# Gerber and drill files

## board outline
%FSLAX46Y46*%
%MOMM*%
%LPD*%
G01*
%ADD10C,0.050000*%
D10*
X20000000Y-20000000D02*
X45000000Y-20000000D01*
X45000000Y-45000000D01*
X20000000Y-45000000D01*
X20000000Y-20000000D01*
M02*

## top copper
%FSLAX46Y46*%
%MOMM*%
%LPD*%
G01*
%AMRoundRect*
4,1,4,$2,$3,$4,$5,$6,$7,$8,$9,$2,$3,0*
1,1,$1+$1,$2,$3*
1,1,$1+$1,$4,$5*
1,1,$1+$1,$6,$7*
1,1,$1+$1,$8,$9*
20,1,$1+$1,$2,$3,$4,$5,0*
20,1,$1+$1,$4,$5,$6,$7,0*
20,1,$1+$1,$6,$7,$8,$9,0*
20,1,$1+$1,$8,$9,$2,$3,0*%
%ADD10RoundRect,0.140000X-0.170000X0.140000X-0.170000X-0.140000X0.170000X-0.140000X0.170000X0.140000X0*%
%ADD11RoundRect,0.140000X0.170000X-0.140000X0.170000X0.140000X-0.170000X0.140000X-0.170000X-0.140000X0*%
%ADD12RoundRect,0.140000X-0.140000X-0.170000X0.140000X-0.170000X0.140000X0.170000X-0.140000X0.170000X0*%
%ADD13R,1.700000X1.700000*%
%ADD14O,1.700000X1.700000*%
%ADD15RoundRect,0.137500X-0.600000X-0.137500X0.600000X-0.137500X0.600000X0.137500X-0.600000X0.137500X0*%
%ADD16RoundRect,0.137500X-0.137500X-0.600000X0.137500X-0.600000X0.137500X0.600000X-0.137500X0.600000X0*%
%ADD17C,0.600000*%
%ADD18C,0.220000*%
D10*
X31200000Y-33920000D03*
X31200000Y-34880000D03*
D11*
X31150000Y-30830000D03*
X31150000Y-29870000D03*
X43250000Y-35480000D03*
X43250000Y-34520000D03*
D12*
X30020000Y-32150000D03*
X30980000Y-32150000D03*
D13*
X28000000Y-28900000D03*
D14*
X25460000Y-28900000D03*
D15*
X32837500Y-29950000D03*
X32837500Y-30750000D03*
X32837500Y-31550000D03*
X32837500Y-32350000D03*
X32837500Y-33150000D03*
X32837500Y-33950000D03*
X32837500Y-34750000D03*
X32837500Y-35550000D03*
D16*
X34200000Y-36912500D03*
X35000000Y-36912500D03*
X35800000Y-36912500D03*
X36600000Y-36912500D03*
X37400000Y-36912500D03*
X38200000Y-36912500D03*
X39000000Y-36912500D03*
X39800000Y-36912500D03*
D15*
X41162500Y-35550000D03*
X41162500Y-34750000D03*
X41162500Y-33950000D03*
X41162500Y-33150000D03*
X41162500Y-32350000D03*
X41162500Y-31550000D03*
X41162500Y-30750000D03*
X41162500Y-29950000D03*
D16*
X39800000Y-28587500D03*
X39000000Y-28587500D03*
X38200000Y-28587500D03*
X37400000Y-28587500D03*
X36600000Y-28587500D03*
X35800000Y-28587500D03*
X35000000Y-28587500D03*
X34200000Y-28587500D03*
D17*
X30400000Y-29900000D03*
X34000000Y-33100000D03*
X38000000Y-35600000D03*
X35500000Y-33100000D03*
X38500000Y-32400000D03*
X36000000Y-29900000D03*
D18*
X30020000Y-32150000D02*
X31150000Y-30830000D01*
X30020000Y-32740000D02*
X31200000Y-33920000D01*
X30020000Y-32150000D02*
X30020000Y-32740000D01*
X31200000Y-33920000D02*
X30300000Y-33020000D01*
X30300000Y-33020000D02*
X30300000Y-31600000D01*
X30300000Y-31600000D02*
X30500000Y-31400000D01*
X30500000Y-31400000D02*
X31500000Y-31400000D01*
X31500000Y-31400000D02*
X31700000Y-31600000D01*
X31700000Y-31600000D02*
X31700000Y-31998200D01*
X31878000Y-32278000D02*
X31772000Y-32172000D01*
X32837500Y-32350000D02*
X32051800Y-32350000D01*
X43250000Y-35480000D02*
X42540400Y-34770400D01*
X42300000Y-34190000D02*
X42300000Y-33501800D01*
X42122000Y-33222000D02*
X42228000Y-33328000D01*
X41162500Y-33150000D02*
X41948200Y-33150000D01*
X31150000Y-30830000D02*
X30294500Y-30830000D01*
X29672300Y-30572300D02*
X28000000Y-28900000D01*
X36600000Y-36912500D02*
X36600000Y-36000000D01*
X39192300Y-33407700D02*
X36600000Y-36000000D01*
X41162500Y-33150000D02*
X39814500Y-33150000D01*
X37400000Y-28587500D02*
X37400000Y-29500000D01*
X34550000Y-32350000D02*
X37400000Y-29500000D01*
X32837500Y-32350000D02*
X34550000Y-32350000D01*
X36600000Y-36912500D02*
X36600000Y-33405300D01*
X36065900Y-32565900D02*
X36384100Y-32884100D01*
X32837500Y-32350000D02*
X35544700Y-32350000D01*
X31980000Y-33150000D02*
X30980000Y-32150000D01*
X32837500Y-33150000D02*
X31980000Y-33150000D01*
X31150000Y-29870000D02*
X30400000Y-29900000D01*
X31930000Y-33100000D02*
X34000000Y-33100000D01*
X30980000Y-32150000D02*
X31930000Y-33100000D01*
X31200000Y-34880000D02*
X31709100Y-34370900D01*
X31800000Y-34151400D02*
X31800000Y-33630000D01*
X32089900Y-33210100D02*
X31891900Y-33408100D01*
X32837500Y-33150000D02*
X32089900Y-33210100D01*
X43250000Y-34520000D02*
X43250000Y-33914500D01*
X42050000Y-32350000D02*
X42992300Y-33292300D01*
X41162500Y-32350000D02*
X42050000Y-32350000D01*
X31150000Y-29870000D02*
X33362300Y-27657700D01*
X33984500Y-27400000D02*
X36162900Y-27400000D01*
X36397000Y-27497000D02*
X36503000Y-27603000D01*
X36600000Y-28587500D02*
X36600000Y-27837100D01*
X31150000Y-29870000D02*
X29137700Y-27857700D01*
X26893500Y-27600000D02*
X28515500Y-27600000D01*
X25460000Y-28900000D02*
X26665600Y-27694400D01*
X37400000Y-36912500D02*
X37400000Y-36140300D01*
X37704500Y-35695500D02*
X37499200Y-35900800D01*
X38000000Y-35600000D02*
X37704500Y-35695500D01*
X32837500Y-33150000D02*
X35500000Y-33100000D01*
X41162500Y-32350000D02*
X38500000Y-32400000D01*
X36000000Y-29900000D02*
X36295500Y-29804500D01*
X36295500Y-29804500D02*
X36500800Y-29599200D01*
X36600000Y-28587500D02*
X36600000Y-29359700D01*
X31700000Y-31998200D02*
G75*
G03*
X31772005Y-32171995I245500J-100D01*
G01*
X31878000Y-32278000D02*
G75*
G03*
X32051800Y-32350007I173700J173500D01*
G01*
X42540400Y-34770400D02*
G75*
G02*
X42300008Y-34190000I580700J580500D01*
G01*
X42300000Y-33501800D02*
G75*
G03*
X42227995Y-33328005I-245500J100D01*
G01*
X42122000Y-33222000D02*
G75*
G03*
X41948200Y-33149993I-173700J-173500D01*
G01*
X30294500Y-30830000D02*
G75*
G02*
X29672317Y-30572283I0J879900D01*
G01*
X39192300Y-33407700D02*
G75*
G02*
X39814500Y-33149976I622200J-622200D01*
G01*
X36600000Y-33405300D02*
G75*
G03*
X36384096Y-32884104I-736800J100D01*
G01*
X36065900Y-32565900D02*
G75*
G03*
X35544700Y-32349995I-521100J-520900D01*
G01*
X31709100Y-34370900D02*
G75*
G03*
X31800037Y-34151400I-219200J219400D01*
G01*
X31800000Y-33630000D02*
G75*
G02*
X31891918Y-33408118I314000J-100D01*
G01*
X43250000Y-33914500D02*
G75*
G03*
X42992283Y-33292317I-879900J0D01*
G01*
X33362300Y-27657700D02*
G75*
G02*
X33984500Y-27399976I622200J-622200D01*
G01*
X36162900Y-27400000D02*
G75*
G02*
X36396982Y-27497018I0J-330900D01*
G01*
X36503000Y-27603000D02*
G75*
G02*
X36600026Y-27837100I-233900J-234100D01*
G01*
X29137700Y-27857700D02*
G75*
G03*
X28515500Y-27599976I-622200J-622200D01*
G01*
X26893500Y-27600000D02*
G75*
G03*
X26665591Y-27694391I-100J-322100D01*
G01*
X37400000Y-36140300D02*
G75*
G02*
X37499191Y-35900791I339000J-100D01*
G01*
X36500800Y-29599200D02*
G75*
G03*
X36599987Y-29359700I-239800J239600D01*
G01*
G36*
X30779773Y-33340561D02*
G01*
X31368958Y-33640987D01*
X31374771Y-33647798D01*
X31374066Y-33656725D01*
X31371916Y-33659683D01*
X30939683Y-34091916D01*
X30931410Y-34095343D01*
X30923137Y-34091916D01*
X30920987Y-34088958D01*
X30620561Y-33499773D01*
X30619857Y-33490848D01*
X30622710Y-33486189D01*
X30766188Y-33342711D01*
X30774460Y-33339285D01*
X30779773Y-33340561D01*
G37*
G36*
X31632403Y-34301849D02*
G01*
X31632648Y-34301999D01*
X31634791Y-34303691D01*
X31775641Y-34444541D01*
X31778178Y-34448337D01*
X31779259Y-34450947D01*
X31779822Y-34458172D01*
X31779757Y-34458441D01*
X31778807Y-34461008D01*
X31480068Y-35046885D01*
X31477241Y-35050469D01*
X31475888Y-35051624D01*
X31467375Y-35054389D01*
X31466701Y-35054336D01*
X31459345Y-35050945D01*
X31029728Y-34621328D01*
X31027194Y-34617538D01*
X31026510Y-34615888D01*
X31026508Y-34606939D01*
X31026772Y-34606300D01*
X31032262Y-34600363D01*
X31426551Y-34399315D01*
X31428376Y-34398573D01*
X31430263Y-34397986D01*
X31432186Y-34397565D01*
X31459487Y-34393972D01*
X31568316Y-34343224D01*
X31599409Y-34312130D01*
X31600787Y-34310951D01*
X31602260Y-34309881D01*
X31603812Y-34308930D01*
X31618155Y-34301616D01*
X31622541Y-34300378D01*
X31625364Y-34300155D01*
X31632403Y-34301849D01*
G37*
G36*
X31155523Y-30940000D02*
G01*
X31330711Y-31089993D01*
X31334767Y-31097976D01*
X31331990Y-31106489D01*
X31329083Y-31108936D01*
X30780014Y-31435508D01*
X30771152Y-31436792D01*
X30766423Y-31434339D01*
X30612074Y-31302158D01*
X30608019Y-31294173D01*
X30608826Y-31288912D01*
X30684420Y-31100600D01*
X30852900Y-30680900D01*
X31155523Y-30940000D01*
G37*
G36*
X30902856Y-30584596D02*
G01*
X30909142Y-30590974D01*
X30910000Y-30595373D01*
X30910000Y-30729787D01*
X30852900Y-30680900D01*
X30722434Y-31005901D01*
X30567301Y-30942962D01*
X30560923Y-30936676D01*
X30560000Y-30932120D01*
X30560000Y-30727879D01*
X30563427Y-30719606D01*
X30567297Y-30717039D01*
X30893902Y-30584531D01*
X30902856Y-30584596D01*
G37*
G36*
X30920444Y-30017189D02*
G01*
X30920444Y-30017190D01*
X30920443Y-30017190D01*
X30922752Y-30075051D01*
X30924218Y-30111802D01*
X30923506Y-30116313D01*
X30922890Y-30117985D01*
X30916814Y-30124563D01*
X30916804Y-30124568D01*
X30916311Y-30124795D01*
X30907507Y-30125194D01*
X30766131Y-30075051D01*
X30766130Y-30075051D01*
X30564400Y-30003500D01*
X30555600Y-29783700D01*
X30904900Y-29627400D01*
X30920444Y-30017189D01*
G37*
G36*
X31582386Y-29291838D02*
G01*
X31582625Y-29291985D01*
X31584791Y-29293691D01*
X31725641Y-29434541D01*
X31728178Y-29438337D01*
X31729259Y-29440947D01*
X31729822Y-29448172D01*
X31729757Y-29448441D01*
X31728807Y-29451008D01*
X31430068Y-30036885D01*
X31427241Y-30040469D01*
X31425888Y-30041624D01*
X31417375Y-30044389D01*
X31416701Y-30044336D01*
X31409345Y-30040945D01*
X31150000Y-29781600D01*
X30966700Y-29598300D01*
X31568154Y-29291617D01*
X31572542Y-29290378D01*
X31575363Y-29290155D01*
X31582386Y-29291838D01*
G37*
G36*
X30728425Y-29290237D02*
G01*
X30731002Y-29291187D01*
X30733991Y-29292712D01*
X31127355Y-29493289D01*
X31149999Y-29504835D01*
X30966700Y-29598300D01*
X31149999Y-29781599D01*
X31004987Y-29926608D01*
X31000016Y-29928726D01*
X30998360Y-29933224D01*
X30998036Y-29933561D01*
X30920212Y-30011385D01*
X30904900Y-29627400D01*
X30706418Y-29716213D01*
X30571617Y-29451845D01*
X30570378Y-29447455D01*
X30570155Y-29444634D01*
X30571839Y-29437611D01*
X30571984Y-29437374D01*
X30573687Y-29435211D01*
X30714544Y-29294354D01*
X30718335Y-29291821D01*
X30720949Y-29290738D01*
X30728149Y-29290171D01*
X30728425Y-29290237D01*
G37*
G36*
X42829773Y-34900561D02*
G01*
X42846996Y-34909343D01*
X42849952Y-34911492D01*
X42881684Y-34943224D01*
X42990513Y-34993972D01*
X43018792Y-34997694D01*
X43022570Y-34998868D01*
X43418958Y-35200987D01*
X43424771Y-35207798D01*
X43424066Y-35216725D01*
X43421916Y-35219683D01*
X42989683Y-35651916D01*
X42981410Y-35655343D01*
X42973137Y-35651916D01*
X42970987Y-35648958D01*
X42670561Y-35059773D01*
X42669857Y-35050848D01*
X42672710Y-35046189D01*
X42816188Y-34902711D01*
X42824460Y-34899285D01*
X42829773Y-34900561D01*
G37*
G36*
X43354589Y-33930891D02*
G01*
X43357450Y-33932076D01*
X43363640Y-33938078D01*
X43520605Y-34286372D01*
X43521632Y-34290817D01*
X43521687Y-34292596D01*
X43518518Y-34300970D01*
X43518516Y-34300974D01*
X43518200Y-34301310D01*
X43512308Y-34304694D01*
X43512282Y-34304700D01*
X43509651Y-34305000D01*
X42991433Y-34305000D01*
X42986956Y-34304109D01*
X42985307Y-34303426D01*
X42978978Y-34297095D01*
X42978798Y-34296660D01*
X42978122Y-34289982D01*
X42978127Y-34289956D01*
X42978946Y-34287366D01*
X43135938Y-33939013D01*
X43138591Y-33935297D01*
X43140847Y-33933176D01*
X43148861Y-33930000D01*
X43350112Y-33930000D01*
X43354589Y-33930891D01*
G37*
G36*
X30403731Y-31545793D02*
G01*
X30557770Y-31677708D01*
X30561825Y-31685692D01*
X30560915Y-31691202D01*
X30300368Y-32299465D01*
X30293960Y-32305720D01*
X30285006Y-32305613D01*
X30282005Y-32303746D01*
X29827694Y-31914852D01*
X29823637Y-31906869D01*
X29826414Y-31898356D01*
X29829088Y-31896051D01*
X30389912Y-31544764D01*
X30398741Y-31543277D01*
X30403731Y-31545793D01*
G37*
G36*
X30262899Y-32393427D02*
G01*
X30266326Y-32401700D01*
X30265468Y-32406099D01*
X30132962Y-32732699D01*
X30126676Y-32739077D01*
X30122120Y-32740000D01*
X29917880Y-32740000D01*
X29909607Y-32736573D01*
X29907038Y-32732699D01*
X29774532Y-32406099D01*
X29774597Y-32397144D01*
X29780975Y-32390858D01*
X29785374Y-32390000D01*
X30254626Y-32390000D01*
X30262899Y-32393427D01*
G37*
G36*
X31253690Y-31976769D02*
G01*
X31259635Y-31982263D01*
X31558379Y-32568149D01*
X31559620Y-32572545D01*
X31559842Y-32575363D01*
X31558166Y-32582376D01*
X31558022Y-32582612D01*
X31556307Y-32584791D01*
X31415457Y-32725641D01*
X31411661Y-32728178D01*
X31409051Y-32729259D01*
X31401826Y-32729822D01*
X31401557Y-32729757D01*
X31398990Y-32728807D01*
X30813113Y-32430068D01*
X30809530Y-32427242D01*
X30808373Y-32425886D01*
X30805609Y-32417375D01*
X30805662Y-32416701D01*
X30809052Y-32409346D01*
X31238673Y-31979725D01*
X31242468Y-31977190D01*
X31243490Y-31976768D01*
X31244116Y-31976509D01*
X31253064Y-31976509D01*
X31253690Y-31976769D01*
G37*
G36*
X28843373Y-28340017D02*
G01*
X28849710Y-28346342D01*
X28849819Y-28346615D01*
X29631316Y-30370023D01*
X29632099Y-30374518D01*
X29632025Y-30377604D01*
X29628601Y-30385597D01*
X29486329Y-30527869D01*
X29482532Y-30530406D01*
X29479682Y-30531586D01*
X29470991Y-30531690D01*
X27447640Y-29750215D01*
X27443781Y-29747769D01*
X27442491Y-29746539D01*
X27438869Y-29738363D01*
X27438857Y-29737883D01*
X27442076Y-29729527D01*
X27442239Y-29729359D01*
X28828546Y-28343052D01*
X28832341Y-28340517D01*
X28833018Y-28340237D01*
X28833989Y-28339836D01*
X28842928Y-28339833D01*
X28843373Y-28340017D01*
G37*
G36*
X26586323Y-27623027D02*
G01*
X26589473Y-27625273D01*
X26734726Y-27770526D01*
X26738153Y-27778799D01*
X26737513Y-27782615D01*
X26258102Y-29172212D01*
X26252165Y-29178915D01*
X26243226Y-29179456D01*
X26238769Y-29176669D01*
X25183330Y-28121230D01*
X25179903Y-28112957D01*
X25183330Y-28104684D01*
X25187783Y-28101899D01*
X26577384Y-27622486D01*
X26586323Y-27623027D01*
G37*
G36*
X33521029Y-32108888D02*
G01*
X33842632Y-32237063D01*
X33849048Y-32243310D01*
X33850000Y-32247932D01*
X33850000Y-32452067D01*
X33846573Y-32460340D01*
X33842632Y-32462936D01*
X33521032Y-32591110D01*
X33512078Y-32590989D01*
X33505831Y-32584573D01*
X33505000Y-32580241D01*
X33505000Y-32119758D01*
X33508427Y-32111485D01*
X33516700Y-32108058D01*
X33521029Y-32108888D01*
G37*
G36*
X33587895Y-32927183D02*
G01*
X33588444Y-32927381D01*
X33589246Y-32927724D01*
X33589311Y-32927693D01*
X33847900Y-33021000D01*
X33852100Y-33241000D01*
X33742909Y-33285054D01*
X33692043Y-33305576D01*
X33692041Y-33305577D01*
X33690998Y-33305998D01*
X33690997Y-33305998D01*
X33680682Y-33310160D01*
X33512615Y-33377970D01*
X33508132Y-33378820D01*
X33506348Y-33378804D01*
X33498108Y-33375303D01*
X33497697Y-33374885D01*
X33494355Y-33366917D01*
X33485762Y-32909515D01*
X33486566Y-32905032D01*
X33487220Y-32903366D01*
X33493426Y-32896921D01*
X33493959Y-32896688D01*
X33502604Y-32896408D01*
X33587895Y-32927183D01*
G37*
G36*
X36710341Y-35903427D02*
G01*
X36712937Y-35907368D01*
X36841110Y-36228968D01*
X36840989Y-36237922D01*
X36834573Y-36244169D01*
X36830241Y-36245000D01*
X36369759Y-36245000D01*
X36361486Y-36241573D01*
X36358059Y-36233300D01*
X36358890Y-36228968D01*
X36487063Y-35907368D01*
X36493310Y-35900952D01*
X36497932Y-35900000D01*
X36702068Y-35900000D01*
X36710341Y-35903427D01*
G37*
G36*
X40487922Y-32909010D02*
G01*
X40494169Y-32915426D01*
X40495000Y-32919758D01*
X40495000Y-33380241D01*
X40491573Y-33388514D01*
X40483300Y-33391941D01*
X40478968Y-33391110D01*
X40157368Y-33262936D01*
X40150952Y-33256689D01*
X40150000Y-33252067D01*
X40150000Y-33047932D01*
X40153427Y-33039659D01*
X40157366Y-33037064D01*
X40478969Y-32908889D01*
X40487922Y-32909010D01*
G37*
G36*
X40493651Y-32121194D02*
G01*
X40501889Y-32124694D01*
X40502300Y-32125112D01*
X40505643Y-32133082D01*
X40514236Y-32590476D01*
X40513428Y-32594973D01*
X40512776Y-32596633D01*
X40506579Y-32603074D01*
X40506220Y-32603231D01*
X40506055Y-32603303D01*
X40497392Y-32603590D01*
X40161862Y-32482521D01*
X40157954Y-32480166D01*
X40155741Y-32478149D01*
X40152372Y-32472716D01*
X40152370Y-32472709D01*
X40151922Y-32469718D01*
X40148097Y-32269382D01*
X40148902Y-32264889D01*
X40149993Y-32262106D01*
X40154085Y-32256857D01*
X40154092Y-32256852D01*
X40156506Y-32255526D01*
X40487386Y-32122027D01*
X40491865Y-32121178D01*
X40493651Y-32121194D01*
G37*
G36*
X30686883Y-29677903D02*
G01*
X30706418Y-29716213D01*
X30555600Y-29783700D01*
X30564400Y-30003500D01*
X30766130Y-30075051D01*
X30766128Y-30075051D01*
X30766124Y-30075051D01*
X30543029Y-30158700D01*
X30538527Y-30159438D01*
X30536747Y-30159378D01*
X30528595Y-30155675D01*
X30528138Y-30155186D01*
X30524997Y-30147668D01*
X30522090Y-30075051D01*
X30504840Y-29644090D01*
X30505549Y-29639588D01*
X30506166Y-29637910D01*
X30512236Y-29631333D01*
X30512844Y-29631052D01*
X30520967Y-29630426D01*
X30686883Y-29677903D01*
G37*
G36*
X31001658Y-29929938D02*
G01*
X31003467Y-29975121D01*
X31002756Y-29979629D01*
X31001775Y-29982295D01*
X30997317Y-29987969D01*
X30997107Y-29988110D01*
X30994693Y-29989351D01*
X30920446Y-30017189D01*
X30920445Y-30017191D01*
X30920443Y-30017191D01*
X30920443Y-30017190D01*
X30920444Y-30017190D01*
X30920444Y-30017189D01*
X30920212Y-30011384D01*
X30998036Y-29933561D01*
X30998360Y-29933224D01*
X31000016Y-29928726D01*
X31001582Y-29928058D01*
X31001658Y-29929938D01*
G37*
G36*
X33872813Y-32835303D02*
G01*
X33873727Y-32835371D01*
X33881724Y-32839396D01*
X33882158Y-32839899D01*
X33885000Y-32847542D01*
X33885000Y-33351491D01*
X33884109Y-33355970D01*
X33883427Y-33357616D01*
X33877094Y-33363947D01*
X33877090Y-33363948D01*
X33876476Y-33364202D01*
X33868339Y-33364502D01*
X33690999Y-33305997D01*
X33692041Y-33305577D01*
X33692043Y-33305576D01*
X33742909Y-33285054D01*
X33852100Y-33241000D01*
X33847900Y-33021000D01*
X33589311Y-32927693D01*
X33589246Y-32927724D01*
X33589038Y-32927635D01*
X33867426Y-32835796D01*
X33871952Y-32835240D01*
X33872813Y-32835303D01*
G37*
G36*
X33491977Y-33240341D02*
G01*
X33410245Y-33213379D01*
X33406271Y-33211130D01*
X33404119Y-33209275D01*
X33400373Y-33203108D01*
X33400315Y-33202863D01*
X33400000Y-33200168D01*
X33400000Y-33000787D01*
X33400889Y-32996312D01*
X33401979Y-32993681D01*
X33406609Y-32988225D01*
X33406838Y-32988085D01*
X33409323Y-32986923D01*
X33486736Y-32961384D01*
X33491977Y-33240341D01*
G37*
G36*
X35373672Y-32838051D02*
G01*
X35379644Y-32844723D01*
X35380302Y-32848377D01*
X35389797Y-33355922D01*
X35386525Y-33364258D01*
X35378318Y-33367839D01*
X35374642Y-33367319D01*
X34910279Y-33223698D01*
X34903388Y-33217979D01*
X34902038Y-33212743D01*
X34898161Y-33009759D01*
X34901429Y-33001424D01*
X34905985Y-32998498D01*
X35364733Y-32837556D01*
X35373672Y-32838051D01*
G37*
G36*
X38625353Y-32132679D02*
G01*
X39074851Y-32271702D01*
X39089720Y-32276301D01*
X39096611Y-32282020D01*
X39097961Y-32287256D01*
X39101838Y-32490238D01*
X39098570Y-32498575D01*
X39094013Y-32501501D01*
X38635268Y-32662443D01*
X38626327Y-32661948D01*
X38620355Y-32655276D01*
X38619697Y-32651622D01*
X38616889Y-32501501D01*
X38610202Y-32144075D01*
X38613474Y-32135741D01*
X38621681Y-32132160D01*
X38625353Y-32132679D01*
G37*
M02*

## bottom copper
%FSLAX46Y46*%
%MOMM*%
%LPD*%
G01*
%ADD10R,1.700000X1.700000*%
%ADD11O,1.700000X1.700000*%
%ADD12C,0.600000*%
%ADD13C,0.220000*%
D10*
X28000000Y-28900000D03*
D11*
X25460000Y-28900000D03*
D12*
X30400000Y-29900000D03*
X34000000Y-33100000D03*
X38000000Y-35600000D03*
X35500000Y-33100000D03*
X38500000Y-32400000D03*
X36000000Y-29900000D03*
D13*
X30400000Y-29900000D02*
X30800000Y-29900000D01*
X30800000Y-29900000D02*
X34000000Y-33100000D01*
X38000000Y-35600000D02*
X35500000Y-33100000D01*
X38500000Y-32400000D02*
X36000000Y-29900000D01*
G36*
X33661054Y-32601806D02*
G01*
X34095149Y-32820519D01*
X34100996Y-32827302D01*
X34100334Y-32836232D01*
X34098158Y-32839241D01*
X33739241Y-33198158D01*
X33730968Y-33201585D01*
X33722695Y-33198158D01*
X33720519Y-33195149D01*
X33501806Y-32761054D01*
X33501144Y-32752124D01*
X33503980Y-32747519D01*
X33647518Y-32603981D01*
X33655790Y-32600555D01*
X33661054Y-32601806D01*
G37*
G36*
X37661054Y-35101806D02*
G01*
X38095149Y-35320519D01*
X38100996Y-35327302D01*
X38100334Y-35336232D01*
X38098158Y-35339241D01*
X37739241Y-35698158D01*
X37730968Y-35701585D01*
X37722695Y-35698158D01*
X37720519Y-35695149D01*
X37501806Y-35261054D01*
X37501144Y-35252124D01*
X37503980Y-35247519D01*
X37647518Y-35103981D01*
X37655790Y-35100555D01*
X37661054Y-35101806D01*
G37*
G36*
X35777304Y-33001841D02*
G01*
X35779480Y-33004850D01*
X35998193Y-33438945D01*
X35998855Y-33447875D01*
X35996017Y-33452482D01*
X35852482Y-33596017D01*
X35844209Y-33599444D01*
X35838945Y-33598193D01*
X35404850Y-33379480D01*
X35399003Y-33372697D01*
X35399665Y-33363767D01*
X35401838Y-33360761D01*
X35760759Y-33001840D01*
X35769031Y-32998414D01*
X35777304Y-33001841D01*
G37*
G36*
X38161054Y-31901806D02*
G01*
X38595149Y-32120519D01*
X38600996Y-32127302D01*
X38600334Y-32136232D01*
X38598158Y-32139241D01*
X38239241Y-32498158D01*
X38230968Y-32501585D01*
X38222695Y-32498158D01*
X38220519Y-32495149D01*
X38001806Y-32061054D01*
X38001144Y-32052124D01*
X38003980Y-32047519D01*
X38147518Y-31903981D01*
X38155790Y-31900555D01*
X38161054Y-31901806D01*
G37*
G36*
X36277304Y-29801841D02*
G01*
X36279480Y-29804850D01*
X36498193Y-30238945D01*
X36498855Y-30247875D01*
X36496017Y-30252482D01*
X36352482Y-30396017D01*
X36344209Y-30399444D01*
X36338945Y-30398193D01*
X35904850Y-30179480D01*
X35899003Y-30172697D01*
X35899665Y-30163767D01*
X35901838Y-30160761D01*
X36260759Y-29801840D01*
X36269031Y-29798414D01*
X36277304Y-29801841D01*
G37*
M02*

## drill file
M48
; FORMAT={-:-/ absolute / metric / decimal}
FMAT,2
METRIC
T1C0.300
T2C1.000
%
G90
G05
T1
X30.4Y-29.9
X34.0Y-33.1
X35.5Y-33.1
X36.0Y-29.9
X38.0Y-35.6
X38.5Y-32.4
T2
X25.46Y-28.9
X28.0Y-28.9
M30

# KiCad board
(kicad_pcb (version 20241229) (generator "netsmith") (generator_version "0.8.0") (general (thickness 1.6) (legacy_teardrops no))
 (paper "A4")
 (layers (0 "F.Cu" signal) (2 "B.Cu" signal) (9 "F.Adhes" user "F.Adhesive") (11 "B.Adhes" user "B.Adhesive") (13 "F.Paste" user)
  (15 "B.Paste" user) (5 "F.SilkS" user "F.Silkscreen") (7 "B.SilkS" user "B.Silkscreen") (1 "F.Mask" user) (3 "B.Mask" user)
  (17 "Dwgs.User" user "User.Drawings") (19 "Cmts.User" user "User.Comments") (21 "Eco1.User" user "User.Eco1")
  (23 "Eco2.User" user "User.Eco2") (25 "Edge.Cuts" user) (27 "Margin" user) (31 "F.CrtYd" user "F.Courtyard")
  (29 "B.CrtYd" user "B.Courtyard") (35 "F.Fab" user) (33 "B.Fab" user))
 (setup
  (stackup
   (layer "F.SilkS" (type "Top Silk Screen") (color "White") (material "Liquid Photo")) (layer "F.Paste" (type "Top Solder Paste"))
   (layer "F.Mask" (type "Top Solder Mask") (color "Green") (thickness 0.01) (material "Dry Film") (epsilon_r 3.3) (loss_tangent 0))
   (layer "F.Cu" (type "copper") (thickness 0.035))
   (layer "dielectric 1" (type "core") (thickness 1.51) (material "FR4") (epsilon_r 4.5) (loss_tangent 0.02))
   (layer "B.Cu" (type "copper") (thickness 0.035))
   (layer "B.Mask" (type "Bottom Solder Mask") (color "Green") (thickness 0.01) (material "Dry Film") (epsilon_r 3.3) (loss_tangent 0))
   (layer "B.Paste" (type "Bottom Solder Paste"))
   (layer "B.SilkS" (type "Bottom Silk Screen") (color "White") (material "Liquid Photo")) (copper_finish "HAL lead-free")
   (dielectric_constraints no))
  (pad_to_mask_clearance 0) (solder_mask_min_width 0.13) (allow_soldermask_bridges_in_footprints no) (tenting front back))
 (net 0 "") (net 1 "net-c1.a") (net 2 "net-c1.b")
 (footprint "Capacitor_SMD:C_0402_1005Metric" (layer "F.Cu") (at 31.2 34.4 270)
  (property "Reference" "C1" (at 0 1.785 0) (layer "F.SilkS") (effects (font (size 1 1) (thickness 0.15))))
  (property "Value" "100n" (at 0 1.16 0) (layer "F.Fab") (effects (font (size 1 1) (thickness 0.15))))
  (pad "1" smd roundrect (at -0.48 0 270) (size 0.56 0.62) (layers "F.Cu" "F.Mask" "F.Paste") (roundrect_rratio 0.25) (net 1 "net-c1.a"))
  (pad "2" smd roundrect (at 0.48 0 270) (size 0.56 0.62) (layers "F.Cu" "F.Mask" "F.Paste") (roundrect_rratio 0.25) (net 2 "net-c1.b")))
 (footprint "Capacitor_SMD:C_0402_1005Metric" (layer "F.Cu") (at 31.15 30.35 90)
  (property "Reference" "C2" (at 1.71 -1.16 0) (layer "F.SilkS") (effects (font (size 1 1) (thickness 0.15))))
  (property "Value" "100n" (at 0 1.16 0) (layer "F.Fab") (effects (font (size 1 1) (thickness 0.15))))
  (pad "1" smd roundrect (at -0.48 0 90) (size 0.56 0.62) (layers "F.Cu" "F.Mask" "F.Paste") (roundrect_rratio 0.25) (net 1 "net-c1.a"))
  (pad "2" smd roundrect (at 0.48 0 90) (size 0.56 0.62) (layers "F.Cu" "F.Mask" "F.Paste") (roundrect_rratio 0.25) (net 2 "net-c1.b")))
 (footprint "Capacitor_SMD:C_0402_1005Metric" (layer "F.Cu") (at 43.25 35 90)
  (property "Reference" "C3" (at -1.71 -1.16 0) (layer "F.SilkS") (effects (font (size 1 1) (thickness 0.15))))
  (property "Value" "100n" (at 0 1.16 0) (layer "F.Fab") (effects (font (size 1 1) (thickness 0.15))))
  (pad "1" smd roundrect (at -0.48 0 90) (size 0.56 0.62) (layers "F.Cu" "F.Mask" "F.Paste") (roundrect_rratio 0.25) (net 1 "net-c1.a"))
  (pad "2" smd roundrect (at 0.48 0 90) (size 0.56 0.62) (layers "F.Cu" "F.Mask" "F.Paste") (roundrect_rratio 0.25) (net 2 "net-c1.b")))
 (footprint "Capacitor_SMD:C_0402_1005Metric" (layer "F.Cu") (at 30.5 32.15)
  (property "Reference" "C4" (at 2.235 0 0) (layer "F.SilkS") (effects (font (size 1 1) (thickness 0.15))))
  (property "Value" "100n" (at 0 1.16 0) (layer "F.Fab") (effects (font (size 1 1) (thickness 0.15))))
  (pad "1" smd roundrect (at -0.48 0) (size 0.56 0.62) (layers "F.Cu" "F.Mask" "F.Paste") (roundrect_rratio 0.25) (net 1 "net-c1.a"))
  (pad "2" smd roundrect (at 0.48 0) (size 0.56 0.62) (layers "F.Cu" "F.Mask" "F.Paste") (roundrect_rratio 0.25) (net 2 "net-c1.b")))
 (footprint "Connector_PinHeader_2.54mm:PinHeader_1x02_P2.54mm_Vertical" (layer "F.Cu") (at 28 28.9 270)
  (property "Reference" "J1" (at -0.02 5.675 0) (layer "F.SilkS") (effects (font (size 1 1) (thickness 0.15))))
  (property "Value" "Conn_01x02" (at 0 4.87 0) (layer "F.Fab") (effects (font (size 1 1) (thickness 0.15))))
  (pad "1" thru_hole rect (at 0 0 270) (size 1.7 1.7) (drill 1) (layers "*.Cu" "*.Mask") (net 1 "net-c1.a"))
  (pad "2" thru_hole oval (at 0 2.54 270) (size 1.7 1.7) (drill 1) (layers "*.Cu" "*.Mask") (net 2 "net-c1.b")))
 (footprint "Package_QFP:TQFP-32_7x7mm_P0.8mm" (layer "F.Cu") (at 37 32.75)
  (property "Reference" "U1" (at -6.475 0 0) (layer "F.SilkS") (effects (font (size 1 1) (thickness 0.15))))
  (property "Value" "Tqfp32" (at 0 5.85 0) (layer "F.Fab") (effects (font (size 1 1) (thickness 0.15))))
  (pad "1" smd roundrect (at -4.1625 -2.8) (size 1.475 0.55) (layers "F.Cu" "F.Mask" "F.Paste") (roundrect_rratio 0.25))
  (pad "2" smd roundrect (at -4.1625 -2) (size 1.475 0.55) (layers "F.Cu" "F.Mask" "F.Paste") (roundrect_rratio 0.25))
  (pad "3" smd roundrect (at -4.1625 -1.2) (size 1.475 0.55) (layers "F.Cu" "F.Mask" "F.Paste") (roundrect_rratio 0.25))
  (pad "4" smd roundrect (at -4.1625 -0.4) (size 1.475 0.55) (layers "F.Cu" "F.Mask" "F.Paste") (roundrect_rratio 0.25) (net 1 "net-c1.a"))
  (pad "5" smd roundrect (at -4.1625 0.4) (size 1.475 0.55) (layers "F.Cu" "F.Mask" "F.Paste") (roundrect_rratio 0.25) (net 2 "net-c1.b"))
  (pad "6" smd roundrect (at -4.1625 1.2) (size 1.475 0.55) (layers "F.Cu" "F.Mask" "F.Paste") (roundrect_rratio 0.25))
  (pad "7" smd roundrect (at -4.1625 2) (size 1.475 0.55) (layers "F.Cu" "F.Mask" "F.Paste") (roundrect_rratio 0.25))
  (pad "8" smd roundrect (at -4.1625 2.8) (size 1.475 0.55) (layers "F.Cu" "F.Mask" "F.Paste") (roundrect_rratio 0.25))
  (pad "9" smd roundrect (at -2.8 4.1625) (size 0.55 1.475) (layers "F.Cu" "F.Mask" "F.Paste") (roundrect_rratio 0.25))
  (pad "10" smd roundrect (at -2 4.1625) (size 0.55 1.475) (layers "F.Cu" "F.Mask" "F.Paste") (roundrect_rratio 0.25))
  (pad "11" smd roundrect (at -1.2 4.1625) (size 0.55 1.475) (layers "F.Cu" "F.Mask" "F.Paste") (roundrect_rratio 0.25))
  (pad "12" smd roundrect (at -0.4 4.1625) (size 0.55 1.475) (layers "F.Cu" "F.Mask" "F.Paste") (roundrect_rratio 0.25) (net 1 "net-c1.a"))
  (pad "13" smd roundrect (at 0.4 4.1625) (size 0.55 1.475) (layers "F.Cu" "F.Mask" "F.Paste") (roundrect_rratio 0.25) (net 2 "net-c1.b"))
  (pad "14" smd roundrect (at 1.2 4.1625) (size 0.55 1.475) (layers "F.Cu" "F.Mask" "F.Paste") (roundrect_rratio 0.25))
  (pad "15" smd roundrect (at 2 4.1625) (size 0.55 1.475) (layers "F.Cu" "F.Mask" "F.Paste") (roundrect_rratio 0.25))
  (pad "16" smd roundrect (at 2.8 4.1625) (size 0.55 1.475) (layers "F.Cu" "F.Mask" "F.Paste") (roundrect_rratio 0.25))
  (pad "17" smd roundrect (at 4.1625 2.8) (size 1.475 0.55) (layers "F.Cu" "F.Mask" "F.Paste") (roundrect_rratio 0.25))
  (pad "18" smd roundrect (at 4.1625 2) (size 1.475 0.55) (layers "F.Cu" "F.Mask" "F.Paste") (roundrect_rratio 0.25))
  (pad "19" smd roundrect (at 4.1625 1.2) (size 1.475 0.55) (layers "F.Cu" "F.Mask" "F.Paste") (roundrect_rratio 0.25))
  (pad "20" smd roundrect (at 4.1625 0.4) (size 1.475 0.55) (layers "F.Cu" "F.Mask" "F.Paste") (roundrect_rratio 0.25) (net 1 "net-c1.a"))
  (pad "21" smd roundrect (at 4.1625 -0.4) (size 1.475 0.55) (layers "F.Cu" "F.Mask" "F.Paste") (roundrect_rratio 0.25) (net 2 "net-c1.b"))
  (pad "22" smd roundrect (at 4.1625 -1.2) (size 1.475 0.55) (layers "F.Cu" "F.Mask" "F.Paste") (roundrect_rratio 0.25))
  (pad "23" smd roundrect (at 4.1625 -2) (size 1.475 0.55) (layers "F.Cu" "F.Mask" "F.Paste") (roundrect_rratio 0.25))
  (pad "24" smd roundrect (at 4.1625 -2.8) (size 1.475 0.55) (layers "F.Cu" "F.Mask" "F.Paste") (roundrect_rratio 0.25))
  (pad "25" smd roundrect (at 2.8 -4.1625) (size 0.55 1.475) (layers "F.Cu" "F.Mask" "F.Paste") (roundrect_rratio 0.25))
  (pad "26" smd roundrect (at 2 -4.1625) (size 0.55 1.475) (layers "F.Cu" "F.Mask" "F.Paste") (roundrect_rratio 0.25))
  (pad "27" smd roundrect (at 1.2 -4.1625) (size 0.55 1.475) (layers "F.Cu" "F.Mask" "F.Paste") (roundrect_rratio 0.25))
  (pad "28" smd roundrect (at 0.4 -4.1625) (size 0.55 1.475) (layers "F.Cu" "F.Mask" "F.Paste") (roundrect_rratio 0.25) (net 1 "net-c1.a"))
  (pad "29" smd roundrect (at -0.4 -4.1625) (size 0.55 1.475) (layers "F.Cu" "F.Mask" "F.Paste") (roundrect_rratio 0.25) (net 2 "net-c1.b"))
  (pad "30" smd roundrect (at -1.2 -4.1625) (size 0.55 1.475) (layers "F.Cu" "F.Mask" "F.Paste") (roundrect_rratio 0.25))
  (pad "31" smd roundrect (at -2 -4.1625) (size 0.55 1.475) (layers "F.Cu" "F.Mask" "F.Paste") (roundrect_rratio 0.25))
  (pad "32" smd roundrect (at -2.8 -4.1625) (size 0.55 1.475) (layers "F.Cu" "F.Mask" "F.Paste") (roundrect_rratio 0.25)))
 (segment (start 30.02 32.15) (end 31.15 30.83) (width 0.22) (layer "F.Cu") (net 1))
 (segment (start 30.02 32.74) (end 31.2 33.92) (width 0.22) (layer "F.Cu") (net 1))
 (segment (start 30.02 32.15) (end 30.02 32.74) (width 0.22) (layer "F.Cu") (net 1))
 (segment (start 31.2 33.92) (end 30.3 33.02) (width 0.22) (layer "F.Cu") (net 1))
 (segment (start 30.3 33.02) (end 30.3 31.6) (width 0.22) (layer "F.Cu") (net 1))
 (segment (start 30.3 31.6) (end 30.5 31.4) (width 0.22) (layer "F.Cu") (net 1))
 (segment (start 30.5 31.4) (end 31.5 31.4) (width 0.22) (layer "F.Cu") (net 1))
 (segment (start 31.5 31.4) (end 31.7 31.6) (width 0.22) (layer "F.Cu") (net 1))
 (segment (start 31.7 31.6) (end 31.7 31.9982) (width 0.22) (layer "F.Cu") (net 1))
 (segment (start 31.878 32.278) (end 31.772 32.172) (width 0.22) (layer "F.Cu") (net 1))
 (segment (start 32.8375 32.35) (end 32.0518 32.35) (width 0.22) (layer "F.Cu") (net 1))
 (segment (start 43.25 35.48) (end 42.5404 34.7704) (width 0.22) (layer "F.Cu") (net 1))
 (segment (start 42.3 34.19) (end 42.3 33.5018) (width 0.22) (layer "F.Cu") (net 1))
 (segment (start 42.122 33.222) (end 42.228 33.328) (width 0.22) (layer "F.Cu") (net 1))
 (segment (start 41.1625 33.15) (end 41.9482 33.15) (width 0.22) (layer "F.Cu") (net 1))
 (segment (start 31.15 30.83) (end 30.2945 30.83) (width 0.22) (layer "F.Cu") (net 1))
 (segment (start 29.6723 30.5723) (end 28 28.9) (width 0.22) (layer "F.Cu") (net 1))
 (segment (start 36.6 36.9125) (end 36.6 36) (width 0.22) (layer "F.Cu") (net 1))
 (segment (start 39.1923 33.4077) (end 36.6 36) (width 0.22) (layer "F.Cu") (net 1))
 (segment (start 41.1625 33.15) (end 39.8145 33.15) (width 0.22) (layer "F.Cu") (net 1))
 (segment (start 37.4 28.5875) (end 37.4 29.5) (width 0.22) (layer "F.Cu") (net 1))
 (segment (start 34.55 32.35) (end 37.4 29.5) (width 0.22) (layer "F.Cu") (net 1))
 (segment (start 32.8375 32.35) (end 34.55 32.35) (width 0.22) (layer "F.Cu") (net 1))
 (segment (start 36.6 36.9125) (end 36.6 33.4053) (width 0.22) (layer "F.Cu") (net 1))
 (segment (start 36.0659 32.5659) (end 36.3841 32.8841) (width 0.22) (layer "F.Cu") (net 1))
 (segment (start 32.8375 32.35) (end 35.5447 32.35) (width 0.22) (layer "F.Cu") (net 1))
 (segment (start 31.98 33.15) (end 30.98 32.15) (width 0.22) (layer "F.Cu") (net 2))
 (segment (start 32.8375 33.15) (end 31.98 33.15) (width 0.22) (layer "F.Cu") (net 2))
 (segment (start 31.15 29.87) (end 30.4 29.9) (width 0.22) (layer "F.Cu") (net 2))
 (segment (start 30.4 29.9) (end 30.8 29.9) (width 0.22) (layer "B.Cu") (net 2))
 (segment (start 30.8 29.9) (end 34 33.1) (width 0.22) (layer "B.Cu") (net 2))
 (segment (start 31.93 33.1) (end 34 33.1) (width 0.22) (layer "F.Cu") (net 2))
 (segment (start 30.98 32.15) (end 31.93 33.1) (width 0.22) (layer "F.Cu") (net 2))
 (segment (start 31.2 34.88) (end 31.7091 34.3709) (width 0.22) (layer "F.Cu") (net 2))
 (segment (start 31.8 34.1514) (end 31.8 33.63) (width 0.22) (layer "F.Cu") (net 2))
 (segment (start 32.0899 33.2101) (end 31.8919 33.4081) (width 0.22) (layer "F.Cu") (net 2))
 (segment (start 32.8375 33.15) (end 32.0899 33.2101) (width 0.22) (layer "F.Cu") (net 2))
 (segment (start 43.25 34.52) (end 43.25 33.9145) (width 0.22) (layer "F.Cu") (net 2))
 (segment (start 42.05 32.35) (end 42.9923 33.2923) (width 0.22) (layer "F.Cu") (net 2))
 (segment (start 41.1625 32.35) (end 42.05 32.35) (width 0.22) (layer "F.Cu") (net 2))
 (segment (start 31.15 29.87) (end 33.3623 27.6577) (width 0.22) (layer "F.Cu") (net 2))
 (segment (start 33.9845 27.4) (end 36.1629 27.4) (width 0.22) (layer "F.Cu") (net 2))
 (segment (start 36.397 27.497) (end 36.503 27.603) (width 0.22) (layer "F.Cu") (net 2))
 (segment (start 36.6 28.5875) (end 36.6 27.8371) (width 0.22) (layer "F.Cu") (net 2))
 (segment (start 31.15 29.87) (end 29.1377 27.8577) (width 0.22) (layer "F.Cu") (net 2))
 (segment (start 26.8935 27.6) (end 28.5155 27.6) (width 0.22) (layer "F.Cu") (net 2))
 (segment (start 25.46 28.9) (end 26.6656 27.6944) (width 0.22) (layer "F.Cu") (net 2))
 (segment (start 37.4 36.9125) (end 37.4 36.1403) (width 0.22) (layer "F.Cu") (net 2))
 (segment (start 37.7045 35.6955) (end 37.4992 35.9008) (width 0.22) (layer "F.Cu") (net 2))
 (segment (start 38 35.6) (end 37.7045 35.6955) (width 0.22) (layer "F.Cu") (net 2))
 (segment (start 38 35.6) (end 35.5 33.1) (width 0.22) (layer "B.Cu") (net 2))
 (segment (start 32.8375 33.15) (end 35.5 33.1) (width 0.22) (layer "F.Cu") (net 2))
 (segment (start 41.1625 32.35) (end 38.5 32.4) (width 0.22) (layer "F.Cu") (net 2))
 (segment (start 38.5 32.4) (end 36 29.9) (width 0.22) (layer "B.Cu") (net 2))
 (segment (start 36 29.9) (end 36.2955 29.8045) (width 0.22) (layer "F.Cu") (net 2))
 (segment (start 36.2955 29.8045) (end 36.5008 29.5992) (width 0.22) (layer "F.Cu") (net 2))
 (segment (start 36.6 28.5875) (end 36.6 29.3597) (width 0.22) (layer "F.Cu") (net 2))
 (arc (start 31.7 31.9982) (mid 31.7187 32.0923) (end 31.772 32.172) (width 0.22) (layer "F.Cu") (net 1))
 (arc (start 31.878 32.278) (mid 31.9577 32.3313) (end 32.0518 32.35) (width 0.22) (layer "F.Cu") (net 1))
 (arc (start 42.5404 34.7704) (mid 42.3625 34.5041) (end 42.3 34.19) (width 0.22) (layer "F.Cu") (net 1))
 (arc (start 42.3 33.5018) (mid 42.2813 33.4077) (end 42.228 33.328) (width 0.22) (layer "F.Cu") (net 1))
 (arc (start 42.122 33.222) (mid 42.0423 33.1687) (end 41.9482 33.15) (width 0.22) (layer "F.Cu") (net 1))
 (arc (start 30.2945 30.83) (mid 29.9577 30.763) (end 29.6723 30.5723) (width 0.22) (layer "F.Cu") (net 1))
 (arc (start 39.1923 33.4077) (mid 39.4777 33.217) (end 39.8145 33.15) (width 0.22) (layer "F.Cu") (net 1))
 (arc (start 36.6 33.4053) (mid 36.5439 33.1232) (end 36.3841 32.8841) (width 0.22) (layer "F.Cu") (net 1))
 (arc (start 36.0659 32.5659) (mid 35.8268 32.4061) (end 35.5447 32.35) (width 0.22) (layer "F.Cu") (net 1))
 (arc (start 31.7091 34.3709) (mid 31.7764 34.2702) (end 31.8 34.1514) (width 0.22) (layer "F.Cu") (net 2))
 (arc (start 31.8 33.63) (mid 31.8239 33.5099) (end 31.8919 33.4081) (width 0.22) (layer "F.Cu") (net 2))
 (arc (start 43.25 33.9145) (mid 43.183 33.5777) (end 42.9923 33.2923) (width 0.22) (layer "F.Cu") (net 2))
 (arc (start 33.3623 27.6577) (mid 33.6477 27.467) (end 33.9845 27.4) (width 0.22) (layer "F.Cu") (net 2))
 (arc (start 36.1629 27.4) (mid 36.2896 27.4252) (end 36.397 27.497) (width 0.22) (layer "F.Cu") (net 2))
 (arc (start 36.503 27.603) (mid 36.5748 27.7104) (end 36.6 27.8371) (width 0.22) (layer "F.Cu") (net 2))
 (arc (start 29.1377 27.8577) (mid 28.8523 27.667) (end 28.5155 27.6) (width 0.22) (layer "F.Cu") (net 2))
 (arc (start 26.8935 27.6) (mid 26.7702 27.6245) (end 26.6656 27.6944) (width 0.22) (layer "F.Cu") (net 2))
 (arc (start 37.4 36.1403) (mid 37.4258 36.0107) (end 37.4992 35.9008) (width 0.22) (layer "F.Cu") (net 2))
 (arc (start 36.5008 29.5992) (mid 36.5742 29.4893) (end 36.6 29.3597) (width 0.22) (layer "F.Cu") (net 2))
 (via (at 30.4 29.9) (size 0.6) (drill 0.3) (layers "F.Cu" "B.Cu") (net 2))
 (via (at 34 33.1) (size 0.6) (drill 0.3) (layers "F.Cu" "B.Cu") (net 2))
 (via (at 38 35.6) (size 0.6) (drill 0.3) (layers "F.Cu" "B.Cu") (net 2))
 (via (at 35.5 33.1) (size 0.6) (drill 0.3) (layers "F.Cu" "B.Cu") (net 2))
 (via (at 38.5 32.4) (size 0.6) (drill 0.3) (layers "F.Cu" "B.Cu") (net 2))
 (via (at 36 29.9) (size 0.6) (drill 0.3) (layers "F.Cu" "B.Cu") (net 2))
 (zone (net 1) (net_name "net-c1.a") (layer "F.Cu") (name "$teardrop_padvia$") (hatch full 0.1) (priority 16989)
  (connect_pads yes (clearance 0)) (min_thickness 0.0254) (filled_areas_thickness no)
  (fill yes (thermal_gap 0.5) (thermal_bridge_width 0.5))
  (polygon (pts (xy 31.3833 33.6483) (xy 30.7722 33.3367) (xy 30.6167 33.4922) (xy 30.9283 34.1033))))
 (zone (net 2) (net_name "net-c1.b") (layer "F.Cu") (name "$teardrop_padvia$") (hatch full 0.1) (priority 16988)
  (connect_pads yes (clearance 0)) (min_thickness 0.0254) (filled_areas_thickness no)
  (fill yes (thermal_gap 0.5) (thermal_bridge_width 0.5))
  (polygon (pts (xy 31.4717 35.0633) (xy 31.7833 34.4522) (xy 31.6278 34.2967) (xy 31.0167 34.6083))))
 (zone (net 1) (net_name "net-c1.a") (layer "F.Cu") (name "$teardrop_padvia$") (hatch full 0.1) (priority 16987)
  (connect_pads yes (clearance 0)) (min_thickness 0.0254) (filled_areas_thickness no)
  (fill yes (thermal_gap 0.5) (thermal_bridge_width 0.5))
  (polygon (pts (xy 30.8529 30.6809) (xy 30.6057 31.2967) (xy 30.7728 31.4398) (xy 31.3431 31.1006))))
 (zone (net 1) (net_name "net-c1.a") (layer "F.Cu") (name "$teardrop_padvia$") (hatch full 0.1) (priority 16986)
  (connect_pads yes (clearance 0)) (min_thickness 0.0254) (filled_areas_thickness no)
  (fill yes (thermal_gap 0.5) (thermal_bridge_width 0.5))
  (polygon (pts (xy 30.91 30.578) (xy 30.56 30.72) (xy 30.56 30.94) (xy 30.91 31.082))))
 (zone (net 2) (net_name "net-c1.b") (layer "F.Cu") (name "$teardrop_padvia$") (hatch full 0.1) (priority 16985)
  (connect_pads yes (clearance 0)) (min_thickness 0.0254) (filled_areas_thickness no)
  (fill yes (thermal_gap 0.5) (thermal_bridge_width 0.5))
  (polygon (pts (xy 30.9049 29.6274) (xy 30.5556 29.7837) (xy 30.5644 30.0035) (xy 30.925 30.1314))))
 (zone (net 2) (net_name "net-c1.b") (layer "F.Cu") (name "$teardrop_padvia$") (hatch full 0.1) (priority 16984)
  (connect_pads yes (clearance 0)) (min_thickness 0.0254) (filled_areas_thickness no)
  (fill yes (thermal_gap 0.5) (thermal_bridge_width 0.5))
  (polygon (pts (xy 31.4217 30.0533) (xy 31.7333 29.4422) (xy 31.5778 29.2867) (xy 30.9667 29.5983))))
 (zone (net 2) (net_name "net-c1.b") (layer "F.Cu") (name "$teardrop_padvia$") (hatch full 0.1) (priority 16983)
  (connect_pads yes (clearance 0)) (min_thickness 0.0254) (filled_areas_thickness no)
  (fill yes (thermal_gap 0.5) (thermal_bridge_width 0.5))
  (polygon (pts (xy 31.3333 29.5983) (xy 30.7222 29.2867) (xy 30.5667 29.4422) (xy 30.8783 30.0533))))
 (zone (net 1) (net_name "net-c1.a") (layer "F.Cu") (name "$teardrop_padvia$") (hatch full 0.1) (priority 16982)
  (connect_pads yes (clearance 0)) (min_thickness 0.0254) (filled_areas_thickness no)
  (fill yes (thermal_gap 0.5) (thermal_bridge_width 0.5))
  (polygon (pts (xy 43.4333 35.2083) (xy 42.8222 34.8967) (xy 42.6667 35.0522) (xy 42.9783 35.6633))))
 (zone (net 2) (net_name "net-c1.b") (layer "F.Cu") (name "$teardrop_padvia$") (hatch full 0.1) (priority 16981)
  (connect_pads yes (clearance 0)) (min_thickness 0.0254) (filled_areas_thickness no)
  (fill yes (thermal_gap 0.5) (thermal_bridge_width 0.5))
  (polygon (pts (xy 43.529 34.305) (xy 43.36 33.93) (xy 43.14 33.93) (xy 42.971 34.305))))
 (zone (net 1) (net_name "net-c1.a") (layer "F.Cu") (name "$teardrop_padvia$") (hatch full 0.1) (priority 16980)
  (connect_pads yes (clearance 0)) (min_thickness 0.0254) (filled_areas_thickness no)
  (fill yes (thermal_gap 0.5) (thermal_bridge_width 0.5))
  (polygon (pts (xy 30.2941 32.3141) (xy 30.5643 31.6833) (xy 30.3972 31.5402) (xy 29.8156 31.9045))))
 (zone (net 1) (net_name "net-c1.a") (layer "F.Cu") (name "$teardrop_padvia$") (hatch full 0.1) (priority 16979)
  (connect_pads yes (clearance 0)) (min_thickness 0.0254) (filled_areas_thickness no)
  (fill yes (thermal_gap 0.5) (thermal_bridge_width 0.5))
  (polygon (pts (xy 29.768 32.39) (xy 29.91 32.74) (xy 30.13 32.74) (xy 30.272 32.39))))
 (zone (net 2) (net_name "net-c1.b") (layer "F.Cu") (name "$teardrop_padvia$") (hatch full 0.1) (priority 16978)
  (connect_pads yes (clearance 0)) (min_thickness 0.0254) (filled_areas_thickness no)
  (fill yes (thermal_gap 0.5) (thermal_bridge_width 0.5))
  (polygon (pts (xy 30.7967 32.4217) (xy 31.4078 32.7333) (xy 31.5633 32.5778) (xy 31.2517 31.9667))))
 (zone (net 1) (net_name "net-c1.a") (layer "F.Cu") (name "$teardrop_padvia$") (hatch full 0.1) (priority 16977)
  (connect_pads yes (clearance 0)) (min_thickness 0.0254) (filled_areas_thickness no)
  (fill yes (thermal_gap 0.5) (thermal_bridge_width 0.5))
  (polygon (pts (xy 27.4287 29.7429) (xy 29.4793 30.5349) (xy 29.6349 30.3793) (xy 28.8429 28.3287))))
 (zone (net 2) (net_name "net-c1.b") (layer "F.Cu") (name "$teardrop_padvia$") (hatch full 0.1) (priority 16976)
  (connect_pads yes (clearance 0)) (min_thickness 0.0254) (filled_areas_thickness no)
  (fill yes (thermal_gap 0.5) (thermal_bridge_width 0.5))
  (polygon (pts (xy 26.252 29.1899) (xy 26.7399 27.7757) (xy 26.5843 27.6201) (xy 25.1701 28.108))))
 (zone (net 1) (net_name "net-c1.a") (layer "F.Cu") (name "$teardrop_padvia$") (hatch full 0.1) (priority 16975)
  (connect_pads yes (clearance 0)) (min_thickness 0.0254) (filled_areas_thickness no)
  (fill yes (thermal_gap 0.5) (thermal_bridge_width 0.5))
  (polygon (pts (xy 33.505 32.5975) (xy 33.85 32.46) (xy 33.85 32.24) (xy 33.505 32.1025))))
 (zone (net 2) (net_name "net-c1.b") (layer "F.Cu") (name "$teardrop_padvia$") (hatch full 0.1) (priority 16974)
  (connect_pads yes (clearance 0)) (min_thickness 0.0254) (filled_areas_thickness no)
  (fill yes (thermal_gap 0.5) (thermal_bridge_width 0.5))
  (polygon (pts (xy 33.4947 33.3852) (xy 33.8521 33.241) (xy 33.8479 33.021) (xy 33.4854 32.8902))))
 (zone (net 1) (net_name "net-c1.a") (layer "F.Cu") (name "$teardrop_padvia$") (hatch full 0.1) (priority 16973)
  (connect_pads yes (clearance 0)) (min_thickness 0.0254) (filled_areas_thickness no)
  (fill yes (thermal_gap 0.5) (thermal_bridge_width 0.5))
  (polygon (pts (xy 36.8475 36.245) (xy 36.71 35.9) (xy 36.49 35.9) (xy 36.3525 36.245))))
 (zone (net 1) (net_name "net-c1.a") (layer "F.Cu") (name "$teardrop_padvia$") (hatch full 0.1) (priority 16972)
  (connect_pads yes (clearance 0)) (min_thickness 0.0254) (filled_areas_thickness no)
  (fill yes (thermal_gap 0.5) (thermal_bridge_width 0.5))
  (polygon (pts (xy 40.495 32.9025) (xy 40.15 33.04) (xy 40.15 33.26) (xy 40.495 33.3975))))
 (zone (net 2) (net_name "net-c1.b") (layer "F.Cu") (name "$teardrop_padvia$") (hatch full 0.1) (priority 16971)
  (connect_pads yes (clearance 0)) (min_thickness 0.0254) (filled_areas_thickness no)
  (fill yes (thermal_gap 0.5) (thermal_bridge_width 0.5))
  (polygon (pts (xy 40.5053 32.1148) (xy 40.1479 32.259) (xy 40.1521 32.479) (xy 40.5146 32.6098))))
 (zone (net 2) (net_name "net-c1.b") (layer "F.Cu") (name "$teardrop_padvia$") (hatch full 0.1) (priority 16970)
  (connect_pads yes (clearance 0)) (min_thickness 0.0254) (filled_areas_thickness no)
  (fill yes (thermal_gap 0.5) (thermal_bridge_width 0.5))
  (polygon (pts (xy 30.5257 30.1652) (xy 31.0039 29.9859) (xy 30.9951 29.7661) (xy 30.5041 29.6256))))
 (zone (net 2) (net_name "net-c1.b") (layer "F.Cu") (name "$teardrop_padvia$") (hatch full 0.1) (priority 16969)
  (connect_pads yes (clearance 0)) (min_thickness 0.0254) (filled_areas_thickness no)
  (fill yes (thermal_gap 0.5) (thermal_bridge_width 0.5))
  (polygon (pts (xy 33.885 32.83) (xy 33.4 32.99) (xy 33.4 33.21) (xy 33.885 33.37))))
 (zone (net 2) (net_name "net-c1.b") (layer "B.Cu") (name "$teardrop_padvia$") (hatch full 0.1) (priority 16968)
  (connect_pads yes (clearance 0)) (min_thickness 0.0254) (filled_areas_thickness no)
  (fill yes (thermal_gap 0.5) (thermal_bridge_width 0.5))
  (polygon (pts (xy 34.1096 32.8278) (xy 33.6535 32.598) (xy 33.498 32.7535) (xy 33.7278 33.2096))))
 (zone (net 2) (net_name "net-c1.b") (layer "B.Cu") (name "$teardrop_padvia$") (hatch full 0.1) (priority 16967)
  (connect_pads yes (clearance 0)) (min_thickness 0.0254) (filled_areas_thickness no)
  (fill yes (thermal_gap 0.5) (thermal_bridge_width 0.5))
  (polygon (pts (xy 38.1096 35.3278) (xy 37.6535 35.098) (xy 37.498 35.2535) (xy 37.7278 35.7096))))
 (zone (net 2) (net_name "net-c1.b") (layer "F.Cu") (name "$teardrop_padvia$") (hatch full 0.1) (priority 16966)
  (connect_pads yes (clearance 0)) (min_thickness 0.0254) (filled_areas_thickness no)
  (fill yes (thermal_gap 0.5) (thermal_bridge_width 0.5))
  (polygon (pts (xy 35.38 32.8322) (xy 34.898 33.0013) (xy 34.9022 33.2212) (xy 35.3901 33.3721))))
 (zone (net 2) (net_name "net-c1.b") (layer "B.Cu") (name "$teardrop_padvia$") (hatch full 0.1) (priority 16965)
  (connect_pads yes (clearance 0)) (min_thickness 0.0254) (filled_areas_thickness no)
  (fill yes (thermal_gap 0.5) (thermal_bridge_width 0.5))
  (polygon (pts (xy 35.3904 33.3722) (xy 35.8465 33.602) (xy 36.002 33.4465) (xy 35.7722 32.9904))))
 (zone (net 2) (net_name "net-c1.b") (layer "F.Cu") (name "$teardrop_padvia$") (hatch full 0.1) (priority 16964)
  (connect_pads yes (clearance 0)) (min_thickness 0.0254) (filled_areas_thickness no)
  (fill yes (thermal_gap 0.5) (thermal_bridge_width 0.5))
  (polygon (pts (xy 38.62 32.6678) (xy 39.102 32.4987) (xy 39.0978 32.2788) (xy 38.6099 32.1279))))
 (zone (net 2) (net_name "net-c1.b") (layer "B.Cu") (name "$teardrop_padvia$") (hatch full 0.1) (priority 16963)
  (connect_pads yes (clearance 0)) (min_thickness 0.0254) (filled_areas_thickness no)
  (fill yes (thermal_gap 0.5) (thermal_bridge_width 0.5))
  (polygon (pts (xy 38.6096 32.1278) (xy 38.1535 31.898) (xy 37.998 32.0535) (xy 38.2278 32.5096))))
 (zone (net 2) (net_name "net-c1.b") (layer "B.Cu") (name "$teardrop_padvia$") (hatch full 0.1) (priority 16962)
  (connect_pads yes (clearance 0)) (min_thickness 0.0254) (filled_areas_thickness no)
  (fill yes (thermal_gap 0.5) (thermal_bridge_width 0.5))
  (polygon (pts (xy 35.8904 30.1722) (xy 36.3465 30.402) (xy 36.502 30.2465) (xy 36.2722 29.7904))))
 (gr_rect (start 20 20) (end 45 45) (stroke (width 0.05) (type default)) (fill no) (layer "Edge.Cuts")))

